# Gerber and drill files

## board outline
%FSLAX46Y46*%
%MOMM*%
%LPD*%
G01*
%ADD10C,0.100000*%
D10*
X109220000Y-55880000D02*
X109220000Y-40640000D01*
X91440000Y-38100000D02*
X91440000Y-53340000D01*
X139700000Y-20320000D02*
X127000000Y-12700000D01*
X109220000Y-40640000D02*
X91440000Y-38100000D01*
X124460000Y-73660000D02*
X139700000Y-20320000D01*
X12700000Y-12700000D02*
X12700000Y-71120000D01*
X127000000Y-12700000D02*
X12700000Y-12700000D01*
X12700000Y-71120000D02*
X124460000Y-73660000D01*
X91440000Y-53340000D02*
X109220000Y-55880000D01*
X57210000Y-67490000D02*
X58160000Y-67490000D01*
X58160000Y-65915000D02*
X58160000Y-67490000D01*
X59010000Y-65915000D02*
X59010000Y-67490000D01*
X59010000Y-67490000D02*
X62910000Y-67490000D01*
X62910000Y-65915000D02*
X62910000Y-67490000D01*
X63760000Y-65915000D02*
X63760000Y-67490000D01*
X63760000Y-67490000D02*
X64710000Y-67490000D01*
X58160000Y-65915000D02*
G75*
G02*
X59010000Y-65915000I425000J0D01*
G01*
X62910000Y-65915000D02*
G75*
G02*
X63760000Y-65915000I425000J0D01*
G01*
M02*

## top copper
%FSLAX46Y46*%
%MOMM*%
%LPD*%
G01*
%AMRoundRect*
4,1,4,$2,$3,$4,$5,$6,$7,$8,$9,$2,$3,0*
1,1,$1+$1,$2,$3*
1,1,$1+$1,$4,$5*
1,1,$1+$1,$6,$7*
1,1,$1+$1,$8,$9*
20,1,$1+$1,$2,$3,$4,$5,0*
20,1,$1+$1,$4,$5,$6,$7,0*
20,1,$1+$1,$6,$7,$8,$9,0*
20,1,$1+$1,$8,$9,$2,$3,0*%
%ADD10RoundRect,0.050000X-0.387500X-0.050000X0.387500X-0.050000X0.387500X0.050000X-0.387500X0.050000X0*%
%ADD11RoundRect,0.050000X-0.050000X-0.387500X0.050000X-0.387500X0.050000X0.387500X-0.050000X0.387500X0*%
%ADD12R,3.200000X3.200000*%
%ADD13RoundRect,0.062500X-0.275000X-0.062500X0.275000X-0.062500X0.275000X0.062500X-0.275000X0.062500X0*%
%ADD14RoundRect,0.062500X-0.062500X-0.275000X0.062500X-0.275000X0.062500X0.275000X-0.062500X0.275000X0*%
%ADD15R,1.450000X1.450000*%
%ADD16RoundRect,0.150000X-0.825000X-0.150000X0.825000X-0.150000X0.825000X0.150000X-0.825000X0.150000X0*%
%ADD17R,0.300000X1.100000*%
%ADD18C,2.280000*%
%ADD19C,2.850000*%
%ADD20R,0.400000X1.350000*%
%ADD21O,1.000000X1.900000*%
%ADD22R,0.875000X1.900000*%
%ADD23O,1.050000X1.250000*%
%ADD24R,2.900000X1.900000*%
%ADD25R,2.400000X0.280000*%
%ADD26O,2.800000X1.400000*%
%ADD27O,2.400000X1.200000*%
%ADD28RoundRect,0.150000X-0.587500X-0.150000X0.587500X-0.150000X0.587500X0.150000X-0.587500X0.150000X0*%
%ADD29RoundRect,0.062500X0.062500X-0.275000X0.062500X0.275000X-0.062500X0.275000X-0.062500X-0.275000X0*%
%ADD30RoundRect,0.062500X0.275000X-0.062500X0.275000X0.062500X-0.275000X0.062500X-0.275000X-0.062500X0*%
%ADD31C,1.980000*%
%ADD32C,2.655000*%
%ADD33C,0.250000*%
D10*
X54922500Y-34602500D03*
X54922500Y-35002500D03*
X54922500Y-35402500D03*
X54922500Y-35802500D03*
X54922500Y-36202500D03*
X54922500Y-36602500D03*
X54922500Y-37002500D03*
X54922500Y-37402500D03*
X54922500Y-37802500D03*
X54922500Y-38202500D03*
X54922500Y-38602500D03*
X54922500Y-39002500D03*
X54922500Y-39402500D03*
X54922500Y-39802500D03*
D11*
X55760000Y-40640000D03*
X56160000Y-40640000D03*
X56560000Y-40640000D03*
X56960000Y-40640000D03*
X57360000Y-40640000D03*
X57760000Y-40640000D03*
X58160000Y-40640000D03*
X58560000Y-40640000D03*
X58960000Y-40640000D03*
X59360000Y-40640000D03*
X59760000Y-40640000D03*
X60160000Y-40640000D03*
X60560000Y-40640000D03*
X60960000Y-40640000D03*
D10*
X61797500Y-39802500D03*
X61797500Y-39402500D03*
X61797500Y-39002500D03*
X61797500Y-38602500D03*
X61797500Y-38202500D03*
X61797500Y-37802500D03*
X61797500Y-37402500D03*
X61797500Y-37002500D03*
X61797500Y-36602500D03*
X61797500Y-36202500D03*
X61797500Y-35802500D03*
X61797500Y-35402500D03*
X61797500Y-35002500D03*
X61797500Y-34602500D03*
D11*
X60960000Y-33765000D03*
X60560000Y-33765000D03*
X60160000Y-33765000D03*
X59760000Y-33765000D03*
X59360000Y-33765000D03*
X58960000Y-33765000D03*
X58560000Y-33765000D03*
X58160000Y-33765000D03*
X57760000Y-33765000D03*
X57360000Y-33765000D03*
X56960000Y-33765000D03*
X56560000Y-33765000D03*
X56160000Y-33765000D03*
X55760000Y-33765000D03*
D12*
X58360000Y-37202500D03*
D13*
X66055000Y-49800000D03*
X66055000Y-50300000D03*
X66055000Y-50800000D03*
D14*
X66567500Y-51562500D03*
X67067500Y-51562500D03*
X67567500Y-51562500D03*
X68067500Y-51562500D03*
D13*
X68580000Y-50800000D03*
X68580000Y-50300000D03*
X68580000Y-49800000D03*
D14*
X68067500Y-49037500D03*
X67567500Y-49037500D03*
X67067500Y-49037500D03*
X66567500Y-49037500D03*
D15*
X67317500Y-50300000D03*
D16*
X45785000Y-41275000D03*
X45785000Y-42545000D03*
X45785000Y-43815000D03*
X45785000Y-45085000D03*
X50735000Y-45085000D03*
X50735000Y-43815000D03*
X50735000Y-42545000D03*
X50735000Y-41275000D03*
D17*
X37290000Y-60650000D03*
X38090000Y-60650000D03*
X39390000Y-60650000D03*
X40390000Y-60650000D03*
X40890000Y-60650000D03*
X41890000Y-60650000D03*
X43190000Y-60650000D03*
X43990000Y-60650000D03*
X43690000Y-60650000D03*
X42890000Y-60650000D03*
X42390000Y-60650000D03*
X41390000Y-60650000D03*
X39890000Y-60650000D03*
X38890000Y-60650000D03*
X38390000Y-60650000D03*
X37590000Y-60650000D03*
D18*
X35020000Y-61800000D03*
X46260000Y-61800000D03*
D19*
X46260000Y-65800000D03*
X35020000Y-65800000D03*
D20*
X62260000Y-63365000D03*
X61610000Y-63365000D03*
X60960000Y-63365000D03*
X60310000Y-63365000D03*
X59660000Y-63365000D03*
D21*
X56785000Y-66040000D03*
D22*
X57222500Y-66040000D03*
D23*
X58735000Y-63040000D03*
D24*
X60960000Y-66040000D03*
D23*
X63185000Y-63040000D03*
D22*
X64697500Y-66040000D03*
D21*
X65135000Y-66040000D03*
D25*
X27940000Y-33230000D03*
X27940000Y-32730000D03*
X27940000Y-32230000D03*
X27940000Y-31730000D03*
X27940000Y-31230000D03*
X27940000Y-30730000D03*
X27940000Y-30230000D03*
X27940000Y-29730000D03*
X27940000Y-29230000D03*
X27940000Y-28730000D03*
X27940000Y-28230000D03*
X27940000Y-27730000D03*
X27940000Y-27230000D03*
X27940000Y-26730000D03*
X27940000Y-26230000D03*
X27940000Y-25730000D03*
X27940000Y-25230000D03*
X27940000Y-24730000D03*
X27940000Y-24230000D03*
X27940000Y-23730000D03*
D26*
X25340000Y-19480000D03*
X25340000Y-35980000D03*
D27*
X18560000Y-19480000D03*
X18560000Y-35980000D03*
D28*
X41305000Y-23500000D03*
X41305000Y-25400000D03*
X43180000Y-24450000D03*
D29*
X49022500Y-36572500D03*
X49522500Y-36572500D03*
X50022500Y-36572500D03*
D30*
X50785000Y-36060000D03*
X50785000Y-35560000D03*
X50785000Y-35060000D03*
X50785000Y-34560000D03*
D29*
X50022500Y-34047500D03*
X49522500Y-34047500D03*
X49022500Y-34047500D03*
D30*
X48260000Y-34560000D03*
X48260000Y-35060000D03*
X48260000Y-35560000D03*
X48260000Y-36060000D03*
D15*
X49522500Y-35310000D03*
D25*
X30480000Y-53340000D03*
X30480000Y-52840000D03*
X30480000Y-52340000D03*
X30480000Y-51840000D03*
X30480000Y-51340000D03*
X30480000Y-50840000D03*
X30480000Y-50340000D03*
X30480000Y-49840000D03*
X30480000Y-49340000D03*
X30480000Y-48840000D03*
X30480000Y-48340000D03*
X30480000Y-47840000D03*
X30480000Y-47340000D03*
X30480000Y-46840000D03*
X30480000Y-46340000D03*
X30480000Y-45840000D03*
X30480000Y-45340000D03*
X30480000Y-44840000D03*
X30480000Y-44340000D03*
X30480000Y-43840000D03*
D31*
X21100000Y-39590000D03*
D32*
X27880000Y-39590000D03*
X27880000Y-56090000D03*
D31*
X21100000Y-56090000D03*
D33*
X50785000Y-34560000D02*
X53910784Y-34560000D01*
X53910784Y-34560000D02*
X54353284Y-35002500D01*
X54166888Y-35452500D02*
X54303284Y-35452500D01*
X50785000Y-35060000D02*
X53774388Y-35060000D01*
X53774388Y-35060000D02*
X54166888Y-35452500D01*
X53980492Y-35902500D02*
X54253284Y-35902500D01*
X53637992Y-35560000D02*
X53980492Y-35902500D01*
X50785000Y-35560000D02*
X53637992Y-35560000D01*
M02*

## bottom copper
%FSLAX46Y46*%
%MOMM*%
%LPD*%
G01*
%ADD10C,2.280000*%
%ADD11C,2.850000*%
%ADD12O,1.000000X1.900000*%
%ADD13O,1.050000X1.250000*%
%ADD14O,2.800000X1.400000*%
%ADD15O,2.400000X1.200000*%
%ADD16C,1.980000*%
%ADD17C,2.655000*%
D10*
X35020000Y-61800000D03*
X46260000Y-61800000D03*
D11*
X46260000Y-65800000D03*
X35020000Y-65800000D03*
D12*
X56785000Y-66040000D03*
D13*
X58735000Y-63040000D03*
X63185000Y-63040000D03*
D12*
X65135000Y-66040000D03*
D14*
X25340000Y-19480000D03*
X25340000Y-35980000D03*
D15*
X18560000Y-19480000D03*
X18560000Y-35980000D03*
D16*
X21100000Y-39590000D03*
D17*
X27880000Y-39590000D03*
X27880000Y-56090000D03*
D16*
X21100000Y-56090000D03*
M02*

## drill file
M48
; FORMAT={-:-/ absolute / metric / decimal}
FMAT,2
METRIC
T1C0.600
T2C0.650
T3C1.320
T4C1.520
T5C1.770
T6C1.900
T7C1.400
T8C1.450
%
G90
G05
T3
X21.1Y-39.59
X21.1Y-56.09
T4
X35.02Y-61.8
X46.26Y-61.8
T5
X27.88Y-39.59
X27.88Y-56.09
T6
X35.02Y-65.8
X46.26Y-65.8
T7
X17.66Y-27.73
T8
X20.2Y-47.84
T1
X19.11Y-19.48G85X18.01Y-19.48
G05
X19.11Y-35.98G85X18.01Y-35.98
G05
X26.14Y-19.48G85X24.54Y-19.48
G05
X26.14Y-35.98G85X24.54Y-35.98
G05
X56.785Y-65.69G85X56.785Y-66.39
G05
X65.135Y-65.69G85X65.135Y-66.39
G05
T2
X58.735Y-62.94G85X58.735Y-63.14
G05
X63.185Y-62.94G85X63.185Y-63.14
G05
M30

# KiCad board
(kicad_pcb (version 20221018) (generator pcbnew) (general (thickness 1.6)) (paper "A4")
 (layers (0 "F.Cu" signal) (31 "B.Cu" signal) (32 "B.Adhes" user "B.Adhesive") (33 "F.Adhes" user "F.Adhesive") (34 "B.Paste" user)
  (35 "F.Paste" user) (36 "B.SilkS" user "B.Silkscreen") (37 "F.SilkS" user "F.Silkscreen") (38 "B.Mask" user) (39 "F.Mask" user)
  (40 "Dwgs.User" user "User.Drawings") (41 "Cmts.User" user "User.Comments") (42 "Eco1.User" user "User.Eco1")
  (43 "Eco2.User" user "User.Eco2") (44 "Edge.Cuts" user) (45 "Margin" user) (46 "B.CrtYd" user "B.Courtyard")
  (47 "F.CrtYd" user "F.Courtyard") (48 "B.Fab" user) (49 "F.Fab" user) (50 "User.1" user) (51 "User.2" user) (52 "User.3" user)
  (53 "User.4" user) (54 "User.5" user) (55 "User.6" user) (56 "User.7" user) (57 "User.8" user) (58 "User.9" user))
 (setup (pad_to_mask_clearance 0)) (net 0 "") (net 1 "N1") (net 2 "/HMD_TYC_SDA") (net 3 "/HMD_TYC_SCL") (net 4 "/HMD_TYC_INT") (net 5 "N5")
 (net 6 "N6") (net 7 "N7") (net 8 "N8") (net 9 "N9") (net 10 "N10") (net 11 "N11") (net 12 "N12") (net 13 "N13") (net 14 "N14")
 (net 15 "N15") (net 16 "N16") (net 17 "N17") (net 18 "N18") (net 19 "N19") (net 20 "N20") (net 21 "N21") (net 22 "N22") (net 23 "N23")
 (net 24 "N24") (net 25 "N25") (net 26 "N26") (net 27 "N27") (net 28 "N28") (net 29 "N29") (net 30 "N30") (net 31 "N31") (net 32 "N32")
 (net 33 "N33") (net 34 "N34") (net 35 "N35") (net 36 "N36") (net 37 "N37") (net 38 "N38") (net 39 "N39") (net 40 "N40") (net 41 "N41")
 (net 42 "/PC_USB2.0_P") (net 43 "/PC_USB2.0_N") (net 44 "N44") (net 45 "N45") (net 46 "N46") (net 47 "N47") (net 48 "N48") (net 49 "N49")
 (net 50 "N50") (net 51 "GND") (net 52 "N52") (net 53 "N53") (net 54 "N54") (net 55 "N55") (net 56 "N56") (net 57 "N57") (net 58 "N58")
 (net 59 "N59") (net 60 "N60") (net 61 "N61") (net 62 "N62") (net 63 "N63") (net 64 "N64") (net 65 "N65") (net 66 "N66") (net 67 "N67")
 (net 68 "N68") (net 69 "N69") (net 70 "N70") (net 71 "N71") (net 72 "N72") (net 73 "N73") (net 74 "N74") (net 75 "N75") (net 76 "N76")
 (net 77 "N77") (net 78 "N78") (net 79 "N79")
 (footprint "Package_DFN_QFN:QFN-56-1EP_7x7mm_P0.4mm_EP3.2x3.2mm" (layer "F.Cu") (at 58.36 37.2025)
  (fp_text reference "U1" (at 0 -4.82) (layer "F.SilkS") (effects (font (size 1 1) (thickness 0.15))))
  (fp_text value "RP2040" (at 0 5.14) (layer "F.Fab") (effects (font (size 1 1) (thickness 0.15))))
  (pad "" smd roundrect (at -0.8 -0.8) (size 1.29 1.29) (layers "F.Paste") (roundrect_rratio 0.193798))
  (pad "" smd roundrect (at -0.8 0.8) (size 1.29 1.29) (layers "F.Paste") (roundrect_rratio 0.193798))
  (pad "" smd roundrect (at 0.8 -0.8) (size 1.29 1.29) (layers "F.Paste") (roundrect_rratio 0.193798))
  (pad "" smd roundrect (at 0.8 0.8) (size 1.29 1.29) (layers "F.Paste") (roundrect_rratio 0.193798))
  (pad "1" smd roundrect (at -3.4375 -2.6) (size 0.875 0.2) (layers "F.Cu" "F.Paste" "F.Mask") (roundrect_rratio 0.25) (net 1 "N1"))
  (pad "2" smd roundrect (at -3.4375 -2.2) (size 0.875 0.2) (layers "F.Cu" "F.Paste" "F.Mask") (roundrect_rratio 0.25)
   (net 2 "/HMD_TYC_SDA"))
  (pad "3" smd roundrect (at -3.4375 -1.8) (size 0.875 0.2) (layers "F.Cu" "F.Paste" "F.Mask") (roundrect_rratio 0.25)
   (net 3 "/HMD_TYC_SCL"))
  (pad "4" smd roundrect (at -3.4375 -1.4) (size 0.875 0.2) (layers "F.Cu" "F.Paste" "F.Mask") (roundrect_rratio 0.25)
   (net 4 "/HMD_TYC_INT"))
  (pad "5" smd roundrect (at -3.4375 -1) (size 0.875 0.2) (layers "F.Cu" "F.Paste" "F.Mask") (roundrect_rratio 0.25) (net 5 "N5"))
  (pad "6" smd roundrect (at -3.4375 -0.6) (size 0.875 0.2) (layers "F.Cu" "F.Paste" "F.Mask") (roundrect_rratio 0.25) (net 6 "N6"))
  (pad "7" smd roundrect (at -3.4375 -0.2) (size 0.875 0.2) (layers "F.Cu" "F.Paste" "F.Mask") (roundrect_rratio 0.25) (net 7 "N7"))
  (pad "8" smd roundrect (at -3.4375 0.2) (size 0.875 0.2) (layers "F.Cu" "F.Paste" "F.Mask") (roundrect_rratio 0.25) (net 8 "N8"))
  (pad "9" smd roundrect (at -3.4375 0.6) (size 0.875 0.2) (layers "F.Cu" "F.Paste" "F.Mask") (roundrect_rratio 0.25) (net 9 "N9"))
  (pad "10" smd roundrect (at -3.4375 1) (size 0.875 0.2) (layers "F.Cu" "F.Paste" "F.Mask") (roundrect_rratio 0.25) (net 1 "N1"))
  (pad "11" smd roundrect (at -3.4375 1.4) (size 0.875 0.2) (layers "F.Cu" "F.Paste" "F.Mask") (roundrect_rratio 0.25) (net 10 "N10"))
  (pad "12" smd roundrect (at -3.4375 1.8) (size 0.875 0.2) (layers "F.Cu" "F.Paste" "F.Mask") (roundrect_rratio 0.25) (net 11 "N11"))
  (pad "13" smd roundrect (at -3.4375 2.2) (size 0.875 0.2) (layers "F.Cu" "F.Paste" "F.Mask") (roundrect_rratio 0.25) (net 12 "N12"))
  (pad "14" smd roundrect (at -3.4375 2.6) (size 0.875 0.2) (layers "F.Cu" "F.Paste" "F.Mask") (roundrect_rratio 0.25) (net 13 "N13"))
  (pad "15" smd roundrect (at -2.6 3.4375) (size 0.2 0.875) (layers "F.Cu" "F.Paste" "F.Mask") (roundrect_rratio 0.25) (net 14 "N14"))
  (pad "16" smd roundrect (at -2.2 3.4375) (size 0.2 0.875) (layers "F.Cu" "F.Paste" "F.Mask") (roundrect_rratio 0.25) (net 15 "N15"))
  (pad "17" smd roundrect (at -1.8 3.4375) (size 0.2 0.875) (layers "F.Cu" "F.Paste" "F.Mask") (roundrect_rratio 0.25) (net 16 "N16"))
  (pad "18" smd roundrect (at -1.4 3.4375) (size 0.2 0.875) (layers "F.Cu" "F.Paste" "F.Mask") (roundrect_rratio 0.25) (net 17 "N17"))
  (pad "19" smd roundrect (at -1 3.4375) (size 0.2 0.875) (layers "F.Cu" "F.Paste" "F.Mask") (roundrect_rratio 0.25) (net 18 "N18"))
  (pad "20" smd roundrect (at -0.6 3.4375) (size 0.2 0.875) (layers "F.Cu" "F.Paste" "F.Mask") (roundrect_rratio 0.25) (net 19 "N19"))
  (pad "21" smd roundrect (at -0.2 3.4375) (size 0.2 0.875) (layers "F.Cu" "F.Paste" "F.Mask") (roundrect_rratio 0.25) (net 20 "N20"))
  (pad "22" smd roundrect (at 0.2 3.4375) (size 0.2 0.875) (layers "F.Cu" "F.Paste" "F.Mask") (roundrect_rratio 0.25) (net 1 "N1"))
  (pad "23" smd roundrect (at 0.6 3.4375) (size 0.2 0.875) (layers "F.Cu" "F.Paste" "F.Mask") (roundrect_rratio 0.25) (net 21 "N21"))
  (pad "24" smd roundrect (at 1 3.4375) (size 0.2 0.875) (layers "F.Cu" "F.Paste" "F.Mask") (roundrect_rratio 0.25) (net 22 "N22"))
  (pad "25" smd roundrect (at 1.4 3.4375) (size 0.2 0.875) (layers "F.Cu" "F.Paste" "F.Mask") (roundrect_rratio 0.25) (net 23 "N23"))
  (pad "26" smd roundrect (at 1.8 3.4375) (size 0.2 0.875) (layers "F.Cu" "F.Paste" "F.Mask") (roundrect_rratio 0.25) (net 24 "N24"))
  (pad "27" smd roundrect (at 2.2 3.4375) (size 0.2 0.875) (layers "F.Cu" "F.Paste" "F.Mask") (roundrect_rratio 0.25) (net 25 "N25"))
  (pad "28" smd roundrect (at 2.6 3.4375) (size 0.2 0.875) (layers "F.Cu" "F.Paste" "F.Mask") (roundrect_rratio 0.25) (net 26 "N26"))
  (pad "29" smd roundrect (at 3.4375 2.6) (size 0.875 0.2) (layers "F.Cu" "F.Paste" "F.Mask") (roundrect_rratio 0.25) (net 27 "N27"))
  (pad "30" smd roundrect (at 3.4375 2.2) (size 0.875 0.2) (layers "F.Cu" "F.Paste" "F.Mask") (roundrect_rratio 0.25) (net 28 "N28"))
  (pad "31" smd roundrect (at 3.4375 1.8) (size 0.875 0.2) (layers "F.Cu" "F.Paste" "F.Mask") (roundrect_rratio 0.25) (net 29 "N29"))
  (pad "32" smd roundrect (at 3.4375 1.4) (size 0.875 0.2) (layers "F.Cu" "F.Paste" "F.Mask") (roundrect_rratio 0.25) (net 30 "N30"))
  (pad "33" smd roundrect (at 3.4375 1) (size 0.875 0.2) (layers "F.Cu" "F.Paste" "F.Mask") (roundrect_rratio 0.25) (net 1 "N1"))
  (pad "34" smd roundrect (at 3.4375 0.6) (size 0.875 0.2) (layers "F.Cu" "F.Paste" "F.Mask") (roundrect_rratio 0.25) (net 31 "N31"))
  (pad "35" smd roundrect (at 3.4375 0.2) (size 0.875 0.2) (layers "F.Cu" "F.Paste" "F.Mask") (roundrect_rratio 0.25) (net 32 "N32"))
  (pad "36" smd roundrect (at 3.4375 -0.2) (size 0.875 0.2) (layers "F.Cu" "F.Paste" "F.Mask") (roundrect_rratio 0.25) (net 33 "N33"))
  (pad "37" smd roundrect (at 3.4375 -0.6) (size 0.875 0.2) (layers "F.Cu" "F.Paste" "F.Mask") (roundrect_rratio 0.25) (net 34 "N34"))
  (pad "38" smd roundrect (at 3.4375 -1) (size 0.875 0.2) (layers "F.Cu" "F.Paste" "F.Mask") (roundrect_rratio 0.25) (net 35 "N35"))
  (pad "39" smd roundrect (at 3.4375 -1.4) (size 0.875 0.2) (layers "F.Cu" "F.Paste" "F.Mask") (roundrect_rratio 0.25) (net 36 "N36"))
  (pad "40" smd roundrect (at 3.4375 -1.8) (size 0.875 0.2) (layers "F.Cu" "F.Paste" "F.Mask") (roundrect_rratio 0.25) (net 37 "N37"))
  (pad "41" smd roundrect (at 3.4375 -2.2) (size 0.875 0.2) (layers "F.Cu" "F.Paste" "F.Mask") (roundrect_rratio 0.25) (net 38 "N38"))
  (pad "42" smd roundrect (at 3.4375 -2.6) (size 0.875 0.2) (layers "F.Cu" "F.Paste" "F.Mask") (roundrect_rratio 0.25) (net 1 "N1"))
  (pad "43" smd roundrect (at 2.6 -3.4375) (size 0.2 0.875) (layers "F.Cu" "F.Paste" "F.Mask") (roundrect_rratio 0.25) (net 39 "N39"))
  (pad "44" smd roundrect (at 2.2 -3.4375) (size 0.2 0.875) (layers "F.Cu" "F.Paste" "F.Mask") (roundrect_rratio 0.25) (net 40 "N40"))
  (pad "45" smd roundrect (at 1.8 -3.4375) (size 0.2 0.875) (layers "F.Cu" "F.Paste" "F.Mask") (roundrect_rratio 0.25) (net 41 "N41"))
  (pad "46" smd roundrect (at 1.4 -3.4375) (size 0.2 0.875) (layers "F.Cu" "F.Paste" "F.Mask") (roundrect_rratio 0.25)
   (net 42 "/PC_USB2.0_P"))
  (pad "47" smd roundrect (at 1 -3.4375) (size 0.2 0.875) (layers "F.Cu" "F.Paste" "F.Mask") (roundrect_rratio 0.25) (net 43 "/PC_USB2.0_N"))
  (pad "48" smd roundrect (at 0.6 -3.4375) (size 0.2 0.875) (layers "F.Cu" "F.Paste" "F.Mask") (roundrect_rratio 0.25) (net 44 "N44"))
  (pad "49" smd roundrect (at 0.2 -3.4375) (size 0.2 0.875) (layers "F.Cu" "F.Paste" "F.Mask") (roundrect_rratio 0.25) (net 1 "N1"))
  (pad "50" smd roundrect (at -0.2 -3.4375) (size 0.2 0.875) (layers "F.Cu" "F.Paste" "F.Mask") (roundrect_rratio 0.25) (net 21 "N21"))
  (pad "51" smd roundrect (at -0.6 -3.4375) (size 0.2 0.875) (layers "F.Cu" "F.Paste" "F.Mask") (roundrect_rratio 0.25) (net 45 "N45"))
  (pad "52" smd roundrect (at -1 -3.4375) (size 0.2 0.875) (layers "F.Cu" "F.Paste" "F.Mask") (roundrect_rratio 0.25) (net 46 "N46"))
  (pad "53" smd roundrect (at -1.4 -3.4375) (size 0.2 0.875) (layers "F.Cu" "F.Paste" "F.Mask") (roundrect_rratio 0.25) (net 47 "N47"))
  (pad "54" smd roundrect (at -1.8 -3.4375) (size 0.2 0.875) (layers "F.Cu" "F.Paste" "F.Mask") (roundrect_rratio 0.25) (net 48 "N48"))
  (pad "55" smd roundrect (at -2.2 -3.4375) (size 0.2 0.875) (layers "F.Cu" "F.Paste" "F.Mask") (roundrect_rratio 0.25) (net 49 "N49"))
  (pad "56" smd roundrect (at -2.6 -3.4375) (size 0.2 0.875) (layers "F.Cu" "F.Paste" "F.Mask") (roundrect_rratio 0.25) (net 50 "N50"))
  (pad "57" smd rect (at 0 0) (size 3.2 3.2) (layers "F.Cu" "F.Mask") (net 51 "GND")))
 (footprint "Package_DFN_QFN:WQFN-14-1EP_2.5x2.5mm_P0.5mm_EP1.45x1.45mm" (layer "F.Cu") (at 67.3175 50.3)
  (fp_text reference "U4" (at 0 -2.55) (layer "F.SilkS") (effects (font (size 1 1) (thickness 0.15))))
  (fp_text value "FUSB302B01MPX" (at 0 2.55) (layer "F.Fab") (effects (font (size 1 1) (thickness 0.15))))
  (pad "" smd roundrect (at -0.36 -0.36) (size 0.58 0.58) (layers "F.Paste") (roundrect_rratio 0.25))
  (pad "" smd roundrect (at -0.36 0.36) (size 0.58 0.58) (layers "F.Paste") (roundrect_rratio 0.25))
  (pad "" smd roundrect (at 0.36 -0.36) (size 0.58 0.58) (layers "F.Paste") (roundrect_rratio 0.25))
  (pad "" smd roundrect (at 0.36 0.36) (size 0.58 0.58) (layers "F.Paste") (roundrect_rratio 0.25))
  (pad "1" smd roundrect (at -1.2625 -0.5) (size 0.675 0.25) (layers "F.Cu" "F.Paste" "F.Mask") (roundrect_rratio 0.25) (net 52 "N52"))
  (pad "2" smd roundrect (at -1.2625 0) (size 0.675 0.25) (layers "F.Cu" "F.Paste" "F.Mask") (roundrect_rratio 0.25) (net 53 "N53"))
  (pad "3" smd roundrect (at -1.2625 0.5) (size 0.675 0.25) (layers "F.Cu" "F.Paste" "F.Mask") (roundrect_rratio 0.25) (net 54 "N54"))
  (pad "4" smd roundrect (at -0.75 1.2625) (size 0.25 0.675) (layers "F.Cu" "F.Paste" "F.Mask") (roundrect_rratio 0.25) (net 54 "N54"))
  (pad "5" smd roundrect (at -0.25 1.2625) (size 0.25 0.675) (layers "F.Cu" "F.Paste" "F.Mask") (roundrect_rratio 0.25) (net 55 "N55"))
  (pad "6" smd roundrect (at 0.25 1.2625) (size 0.25 0.675) (layers "F.Cu" "F.Paste" "F.Mask") (roundrect_rratio 0.25) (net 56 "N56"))
  (pad "7" smd roundrect (at 0.75 1.2625) (size 0.25 0.675) (layers "F.Cu" "F.Paste" "F.Mask") (roundrect_rratio 0.25) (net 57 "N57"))
  (pad "8" smd roundrect (at 1.2625 0.5) (size 0.675 0.25) (layers "F.Cu" "F.Paste" "F.Mask") (roundrect_rratio 0.25) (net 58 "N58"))
  (pad "9" smd roundrect (at 1.2625 0) (size 0.675 0.25) (layers "F.Cu" "F.Paste" "F.Mask") (roundrect_rratio 0.25) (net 58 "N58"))
  (pad "10" smd roundrect (at 1.2625 -0.5) (size 0.675 0.25) (layers "F.Cu" "F.Paste" "F.Mask") (roundrect_rratio 0.25) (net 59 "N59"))
  (pad "11" smd roundrect (at 0.75 -1.2625) (size 0.25 0.675) (layers "F.Cu" "F.Paste" "F.Mask") (roundrect_rratio 0.25) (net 59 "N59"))
  (pad "12" smd roundrect (at 0.25 -1.2625) (size 0.25 0.675) (layers "F.Cu" "F.Paste" "F.Mask") (roundrect_rratio 0.25) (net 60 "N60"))
  (pad "13" smd roundrect (at -0.25 -1.2625) (size 0.25 0.675) (layers "F.Cu" "F.Paste" "F.Mask") (roundrect_rratio 0.25) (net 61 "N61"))
  (pad "14" smd roundrect (at -0.75 -1.2625) (size 0.25 0.675) (layers "F.Cu" "F.Paste" "F.Mask") (roundrect_rratio 0.25) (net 52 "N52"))
  (pad "15" smd rect (at 0 0) (size 1.45 1.45) (layers "F.Cu" "F.Mask") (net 58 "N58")))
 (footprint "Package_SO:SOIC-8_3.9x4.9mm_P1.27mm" (layer "F.Cu") (at 48.26 43.18)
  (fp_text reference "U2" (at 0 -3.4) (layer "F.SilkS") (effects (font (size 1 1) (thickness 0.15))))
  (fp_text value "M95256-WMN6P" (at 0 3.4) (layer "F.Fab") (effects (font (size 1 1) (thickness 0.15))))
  (pad "1" smd roundrect (at -2.475 -1.905) (size 1.95 0.6) (layers "F.Cu" "F.Paste" "F.Mask") (roundrect_rratio 0.25) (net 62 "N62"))
  (pad "2" smd roundrect (at -2.475 -0.635) (size 1.95 0.6) (layers "F.Cu" "F.Paste" "F.Mask") (roundrect_rratio 0.25) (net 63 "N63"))
  (pad "3" smd roundrect (at -2.475 0.635) (size 1.95 0.6) (layers "F.Cu" "F.Paste" "F.Mask") (roundrect_rratio 0.25) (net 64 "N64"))
  (pad "4" smd roundrect (at -2.475 1.905) (size 1.95 0.6) (layers "F.Cu" "F.Paste" "F.Mask") (roundrect_rratio 0.25) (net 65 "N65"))
  (pad "5" smd roundrect (at 2.475 1.905) (size 1.95 0.6) (layers "F.Cu" "F.Paste" "F.Mask") (roundrect_rratio 0.25) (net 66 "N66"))
  (pad "6" smd roundrect (at 2.475 0.635) (size 1.95 0.6) (layers "F.Cu" "F.Paste" "F.Mask") (roundrect_rratio 0.25) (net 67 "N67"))
  (pad "7" smd roundrect (at 2.475 -0.635) (size 1.95 0.6) (layers "F.Cu" "F.Paste" "F.Mask") (roundrect_rratio 0.25) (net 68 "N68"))
  (pad "8" smd roundrect (at 2.475 -1.905) (size 1.95 0.6) (layers "F.Cu" "F.Paste" "F.Mask") (roundrect_rratio 0.25) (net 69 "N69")))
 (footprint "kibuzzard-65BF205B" (layer "F.Cu") (at 88.9 27.94)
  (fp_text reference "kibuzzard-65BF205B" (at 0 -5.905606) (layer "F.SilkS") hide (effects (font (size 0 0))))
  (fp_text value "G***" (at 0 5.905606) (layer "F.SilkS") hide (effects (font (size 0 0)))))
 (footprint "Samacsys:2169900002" (layer "F.Cu") (at 40.64 63.5)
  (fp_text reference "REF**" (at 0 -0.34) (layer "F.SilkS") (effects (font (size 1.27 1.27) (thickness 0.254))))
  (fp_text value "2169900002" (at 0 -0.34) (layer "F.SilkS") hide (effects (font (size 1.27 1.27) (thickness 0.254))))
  (pad "A1" smd rect (at -3.35 -2.85) (size 0.3 1.1) (layers "F.Cu" "F.Paste" "F.Mask"))
  (pad "A4" smd rect (at -2.55 -2.85) (size 0.3 1.1) (layers "F.Cu" "F.Paste" "F.Mask"))
  (pad "A5" smd rect (at -1.25 -2.85) (size 0.3 1.1) (layers "F.Cu" "F.Paste" "F.Mask"))
  (pad "A6" smd rect (at -0.25 -2.85) (size 0.3 1.1) (layers "F.Cu" "F.Paste" "F.Mask"))
  (pad "A7" smd rect (at 0.25 -2.85) (size 0.3 1.1) (layers "F.Cu" "F.Paste" "F.Mask"))
  (pad "A8" smd rect (at 1.25 -2.85) (size 0.3 1.1) (layers "F.Cu" "F.Paste" "F.Mask"))
  (pad "A9" smd rect (at 2.55 -2.85) (size 0.3 1.1) (layers "F.Cu" "F.Paste" "F.Mask"))
  (pad "A12" smd rect (at 3.35 -2.85) (size 0.3 1.1) (layers "F.Cu" "F.Paste" "F.Mask"))
  (pad "B1" smd rect (at 3.05 -2.85) (size 0.3 1.1) (layers "F.Cu" "F.Paste" "F.Mask"))
  (pad "B4" smd rect (at 2.25 -2.85) (size 0.3 1.1) (layers "F.Cu" "F.Paste" "F.Mask"))
  (pad "B5" smd rect (at 1.75 -2.85) (size 0.3 1.1) (layers "F.Cu" "F.Paste" "F.Mask"))
  (pad "B6" smd rect (at 0.75 -2.85) (size 0.3 1.1) (layers "F.Cu" "F.Paste" "F.Mask"))
  (pad "B7" smd rect (at -0.75 -2.85) (size 0.3 1.1) (layers "F.Cu" "F.Paste" "F.Mask"))
  (pad "B8" smd rect (at -1.75 -2.85) (size 0.3 1.1) (layers "F.Cu" "F.Paste" "F.Mask"))
  (pad "B9" smd rect (at -2.25 -2.85) (size 0.3 1.1) (layers "F.Cu" "F.Paste" "F.Mask"))
  (pad "B12" smd rect (at -3.05 -2.85) (size 0.3 1.1) (layers "F.Cu" "F.Paste" "F.Mask"))
  (pad "MH1" thru_hole circle (at -5.62 -1.7) (size 2.28 2.28) (drill 1.52) (layers "*.Cu" "*.Mask"))
  (pad "MH2" thru_hole circle (at 5.62 -1.7) (size 2.28 2.28) (drill 1.52) (layers "*.Cu" "*.Mask"))
  (pad "MH3" thru_hole circle (at 5.62 2.3) (size 2.85 2.85) (drill 1.9) (layers "*.Cu" "*.Mask"))
  (pad "MH4" thru_hole circle (at -5.62 2.3) (size 2.85 2.85) (drill 1.9) (layers "*.Cu" "*.Mask")))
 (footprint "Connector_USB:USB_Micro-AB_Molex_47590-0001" (layer "F.Cu") (at 60.96 66.04)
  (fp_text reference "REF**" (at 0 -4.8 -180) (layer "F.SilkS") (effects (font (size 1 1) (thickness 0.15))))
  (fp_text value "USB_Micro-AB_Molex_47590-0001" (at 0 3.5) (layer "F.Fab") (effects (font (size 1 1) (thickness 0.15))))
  (fp_line (start -3.75 1.45) (end -2.8 1.45) (stroke (width 0.1) (type solid)) (layer "Edge.Cuts"))
  (fp_line (start -2.8 -0.125) (end -2.8 1.45) (stroke (width 0.1) (type solid)) (layer "Edge.Cuts"))
  (fp_line (start -1.95 -0.125) (end -1.95 1.45) (stroke (width 0.1) (type solid)) (layer "Edge.Cuts"))
  (fp_line (start -1.95 1.45) (end 1.95 1.45) (stroke (width 0.1) (type solid)) (layer "Edge.Cuts"))
  (fp_line (start 1.95 -0.125) (end 1.95 1.45) (stroke (width 0.1) (type solid)) (layer "Edge.Cuts"))
  (fp_line (start 2.8 -0.125) (end 2.8 1.45) (stroke (width 0.1) (type solid)) (layer "Edge.Cuts"))
  (fp_line (start 2.8 1.45) (end 3.75 1.45) (stroke (width 0.1) (type solid)) (layer "Edge.Cuts"))
  (fp_arc (start -2.8 -0.125) (mid -2.375 -0.55) (end -1.95 -0.125) (stroke (width 0.1) (type solid)) (layer "Edge.Cuts"))
  (fp_arc (start 1.95 -0.125) (mid 2.375 -0.55) (end 2.8 -0.125) (stroke (width 0.1) (type solid)) (layer "Edge.Cuts"))
  (pad "" smd rect (at -3.5 0) (size 0.3 0.85) (layers "F.Paste"))
  (pad "" smd rect (at 3.5 0) (size 0.3 0.85) (layers "F.Paste"))
  (pad "1" smd rect (at 1.3 -2.675) (size 0.4 1.35) (layers "F.Cu" "F.Paste" "F.Mask"))
  (pad "2" smd rect (at 0.65 -2.675) (size 0.4 1.35) (layers "F.Cu" "F.Paste" "F.Mask"))
  (pad "3" smd rect (at 0 -2.675) (size 0.4 1.35) (layers "F.Cu" "F.Paste" "F.Mask"))
  (pad "4" smd rect (at -0.65 -2.675) (size 0.4 1.35) (layers "F.Cu" "F.Paste" "F.Mask"))
  (pad "5" smd rect (at -1.3 -2.675) (size 0.4 1.35) (layers "F.Cu" "F.Paste" "F.Mask"))
  (pad "6" thru_hole oval (at -4.175 0) (size 1 1.9) (drill oval 0.6 1.3) (layers "*.Cu" "*.Mask"))
  (pad "6" smd rect (at -3.7375 0) (size 0.875 1.9) (layers "F.Cu" "F.Mask"))
  (pad "6" thru_hole oval (at -2.225 -3) (size 1.05 1.25) (drill oval 0.65 0.85) (layers "*.Cu" "*.Mask"))
  (pad "6" smd rect (at 0 0) (size 2.9 1.9) (layers "F.Cu" "F.Paste" "F.Mask"))
  (pad "6" thru_hole oval (at 2.225 -3) (size 1.05 1.25) (drill oval 0.65 0.85) (layers "*.Cu" "*.Mask"))
  (pad "6" smd rect (at 3.7375 0) (size 0.875 1.9) (layers "F.Cu" "F.Mask"))
  (pad "6" thru_hole oval (at 4.175 0) (size 1 1.9) (drill oval 0.6 1.3) (layers "*.Cu" "*.Mask")))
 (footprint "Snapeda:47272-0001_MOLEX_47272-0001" (layer "F.Cu") (at 14.38 27.73 -90)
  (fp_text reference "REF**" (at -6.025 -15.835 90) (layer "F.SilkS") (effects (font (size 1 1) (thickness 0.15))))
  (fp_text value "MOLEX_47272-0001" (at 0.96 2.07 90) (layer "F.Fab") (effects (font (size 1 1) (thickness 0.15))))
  (pad "" np_thru_hole circle (at 0 -3.28 270) (size 1.4 1.4) (drill 1.4) (layers "*.Cu" "*.Mask"))
  (pad "1" smd rect (at 5.5 -13.56) (size 2.4 0.28) (layers "F.Cu" "F.Paste" "F.Mask") (solder_mask_margin 0.0762))
  (pad "2" smd rect (at 5 -13.56) (size 2.4 0.28) (layers "F.Cu" "F.Paste" "F.Mask") (solder_mask_margin 0.0762))
  (pad "3" smd rect (at 4.5 -13.56) (size 2.4 0.28) (layers "F.Cu" "F.Paste" "F.Mask") (solder_mask_margin 0.0762))
  (pad "4" smd rect (at 4 -13.56) (size 2.4 0.28) (layers "F.Cu" "F.Paste" "F.Mask") (solder_mask_margin 0.0762))
  (pad "5" smd rect (at 3.5 -13.56) (size 2.4 0.28) (layers "F.Cu" "F.Paste" "F.Mask") (solder_mask_margin 0.0762))
  (pad "6" smd rect (at 3 -13.56) (size 2.4 0.28) (layers "F.Cu" "F.Paste" "F.Mask") (solder_mask_margin 0.0762))
  (pad "7" smd rect (at 2.5 -13.56) (size 2.4 0.28) (layers "F.Cu" "F.Paste" "F.Mask") (solder_mask_margin 0.0762))
  (pad "8" smd rect (at 2 -13.56) (size 2.4 0.28) (layers "F.Cu" "F.Paste" "F.Mask") (solder_mask_margin 0.0762))
  (pad "9" smd rect (at 1.5 -13.56) (size 2.4 0.28) (layers "F.Cu" "F.Paste" "F.Mask") (solder_mask_margin 0.0762))
  (pad "10" smd rect (at 1 -13.56) (size 2.4 0.28) (layers "F.Cu" "F.Paste" "F.Mask") (solder_mask_margin 0.0762))
  (pad "11" smd rect (at 0.5 -13.56) (size 2.4 0.28) (layers "F.Cu" "F.Paste" "F.Mask") (solder_mask_margin 0.0762))
  (pad "12" smd rect (at 0 -13.56) (size 2.4 0.28) (layers "F.Cu" "F.Paste" "F.Mask") (solder_mask_margin 0.0762))
  (pad "13" smd rect (at -0.5 -13.56) (size 2.4 0.28) (layers "F.Cu" "F.Paste" "F.Mask") (solder_mask_margin 0.0762))
  (pad "14" smd rect (at -1 -13.56) (size 2.4 0.28) (layers "F.Cu" "F.Paste" "F.Mask") (solder_mask_margin 0.0762))
  (pad "15" smd rect (at -1.5 -13.56) (size 2.4 0.28) (layers "F.Cu" "F.Paste" "F.Mask") (solder_mask_margin 0.0762))
  (pad "16" smd rect (at -2 -13.56) (size 2.4 0.28) (layers "F.Cu" "F.Paste" "F.Mask") (solder_mask_margin 0.0762))
  (pad "17" smd rect (at -2.5 -13.56) (size 2.4 0.28) (layers "F.Cu" "F.Paste" "F.Mask") (solder_mask_margin 0.0762))
  (pad "18" smd rect (at -3 -13.56) (size 2.4 0.28) (layers "F.Cu" "F.Paste" "F.Mask") (solder_mask_margin 0.0762))
  (pad "19" smd rect (at -3.5 -13.56) (size 2.4 0.28) (layers "F.Cu" "F.Paste" "F.Mask") (solder_mask_margin 0.0762))
  (pad "20" smd rect (at -4 -13.56) (size 2.4 0.28) (layers "F.Cu" "F.Paste" "F.Mask") (solder_mask_margin 0.0762))
  (pad "S1" thru_hole oval (at -8.25 -10.96 270) (size 1.4 2.8) (drill oval 0.6 2.2) (layers "*.Cu" "*.Mask") (solder_mask_margin 0.0762))
  (pad "S2" thru_hole oval (at 8.25 -10.96 270) (size 1.4 2.8) (drill oval 0.6 2.2) (layers "*.Cu" "*.Mask") (solder_mask_margin 0.0762))
  (pad "S3" thru_hole oval (at -8.25 -4.18 270) (size 1.2 2.4) (drill oval 0.6 1.7) (layers "*.Cu" "*.Mask") (solder_mask_margin 0.0762))
  (pad "S4" thru_hole oval (at 8.25 -4.18 270) (size 1.2 2.4) (drill oval 0.6 1.7) (layers "*.Cu" "*.Mask") (solder_mask_margin 0.0762)))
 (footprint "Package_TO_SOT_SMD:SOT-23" (layer "F.Cu") (at 42.2425 24.45)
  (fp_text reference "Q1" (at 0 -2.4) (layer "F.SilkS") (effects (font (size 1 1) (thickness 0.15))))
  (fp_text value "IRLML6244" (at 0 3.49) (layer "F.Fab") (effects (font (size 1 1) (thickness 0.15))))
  (pad "1" smd roundrect (at -0.9375 -0.95) (size 1.475 0.6) (layers "F.Cu" "F.Paste" "F.Mask") (roundrect_rratio 0.25) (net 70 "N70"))
  (pad "2" smd roundrect (at -0.9375 0.95) (size 1.475 0.6) (layers "F.Cu" "F.Paste" "F.Mask") (roundrect_rratio 0.25) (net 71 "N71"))
  (pad "3" smd roundrect (at 0.9375 0) (size 1.475 0.6) (layers "F.Cu" "F.Paste" "F.Mask") (roundrect_rratio 0.25) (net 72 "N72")))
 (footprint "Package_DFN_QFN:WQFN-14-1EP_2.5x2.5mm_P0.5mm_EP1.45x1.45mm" (layer "F.Cu") (at 49.5225 35.31 90)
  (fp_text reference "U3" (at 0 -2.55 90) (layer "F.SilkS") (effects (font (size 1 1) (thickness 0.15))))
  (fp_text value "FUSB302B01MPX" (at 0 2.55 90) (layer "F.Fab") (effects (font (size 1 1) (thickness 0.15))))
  (pad "" smd roundrect (at -0.36 -0.36 90) (size 0.58 0.58) (layers "F.Paste") (roundrect_rratio 0.25))
  (pad "" smd roundrect (at -0.36 0.36 90) (size 0.58 0.58) (layers "F.Paste") (roundrect_rratio 0.25))
  (pad "" smd roundrect (at 0.36 -0.36 90) (size 0.58 0.58) (layers "F.Paste") (roundrect_rratio 0.25))
  (pad "" smd roundrect (at 0.36 0.36 90) (size 0.58 0.58) (layers "F.Paste") (roundrect_rratio 0.25))
  (pad "1" smd roundrect (at -1.2625 -0.5 90) (size 0.675 0.25) (layers "F.Cu" "F.Paste" "F.Mask") (roundrect_rratio 0.25) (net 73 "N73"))
  (pad "2" smd roundrect (at -1.2625 0 90) (size 0.675 0.25) (layers "F.Cu" "F.Paste" "F.Mask") (roundrect_rratio 0.25) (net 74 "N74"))
  (pad "3" smd roundrect (at -1.2625 0.5 90) (size 0.675 0.25) (layers "F.Cu" "F.Paste" "F.Mask") (roundrect_rratio 0.25) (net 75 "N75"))
  (pad "4" smd roundrect (at -0.75 1.2625 90) (size 0.25 0.675) (layers "F.Cu" "F.Paste" "F.Mask") (roundrect_rratio 0.25) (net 75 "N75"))
  (pad "5" smd roundrect (at -0.25 1.2625 90) (size 0.25 0.675) (layers "F.Cu" "F.Paste" "F.Mask") (roundrect_rratio 0.25)
   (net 4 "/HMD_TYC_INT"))
  (pad "6" smd roundrect (at 0.25 1.2625 90) (size 0.25 0.675) (layers "F.Cu" "F.Paste" "F.Mask") (roundrect_rratio 0.25)
   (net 3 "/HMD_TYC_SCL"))
  (pad "7" smd roundrect (at 0.75 1.2625 90) (size 0.25 0.675) (layers "F.Cu" "F.Paste" "F.Mask") (roundrect_rratio 0.25)
   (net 2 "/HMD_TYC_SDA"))
  (pad "8" smd roundrect (at 1.2625 0.5 90) (size 0.675 0.25) (layers "F.Cu" "F.Paste" "F.Mask") (roundrect_rratio 0.25) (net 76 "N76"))
  (pad "9" smd roundrect (at 1.2625 0 90) (size 0.675 0.25) (layers "F.Cu" "F.Paste" "F.Mask") (roundrect_rratio 0.25) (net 76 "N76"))
  (pad "10" smd roundrect (at 1.2625 -0.5 90) (size 0.675 0.25) (layers "F.Cu" "F.Paste" "F.Mask") (roundrect_rratio 0.25) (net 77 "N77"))
  (pad "11" smd roundrect (at 0.75 -1.2625 90) (size 0.25 0.675) (layers "F.Cu" "F.Paste" "F.Mask") (roundrect_rratio 0.25) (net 77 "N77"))
  (pad "12" smd roundrect (at 0.25 -1.2625 90) (size 0.25 0.675) (layers "F.Cu" "F.Paste" "F.Mask") (roundrect_rratio 0.25) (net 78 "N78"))
  (pad "13" smd roundrect (at -0.25 -1.2625 90) (size 0.25 0.675) (layers "F.Cu" "F.Paste" "F.Mask") (roundrect_rratio 0.25) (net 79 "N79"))
  (pad "14" smd roundrect (at -0.75 -1.2625 90) (size 0.25 0.675) (layers "F.Cu" "F.Paste" "F.Mask") (roundrect_rratio 0.25) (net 73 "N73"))
  (pad "15" smd rect (at 0 0 90) (size 1.45 1.45) (layers "F.Cu" "F.Mask") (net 76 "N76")))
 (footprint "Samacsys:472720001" (layer "F.Cu") (at 23.19 47.84 -90)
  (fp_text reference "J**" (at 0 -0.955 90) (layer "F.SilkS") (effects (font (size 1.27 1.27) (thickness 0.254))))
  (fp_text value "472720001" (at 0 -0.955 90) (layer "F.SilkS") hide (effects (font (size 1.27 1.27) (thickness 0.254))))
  (pad "" np_thru_hole circle (at 0 2.99 270) (size 1.45 1.45) (drill 1.45) (layers "*.Cu" "*.Mask"))
  (pad "1" smd rect (at 5.5 -7.29 270) (size 0.28 2.4) (layers "F.Cu" "F.Paste" "F.Mask"))
  (pad "2" smd rect (at 5 -7.29 270) (size 0.28 2.4) (layers "F.Cu" "F.Paste" "F.Mask"))
  (pad "3" smd rect (at 4.5 -7.29 270) (size 0.28 2.4) (layers "F.Cu" "F.Paste" "F.Mask"))
  (pad "4" smd rect (at 4 -7.29 270) (size 0.28 2.4) (layers "F.Cu" "F.Paste" "F.Mask"))
  (pad "5" smd rect (at 3.5 -7.29 270) (size 0.28 2.4) (layers "F.Cu" "F.Paste" "F.Mask"))
  (pad "6" smd rect (at 3 -7.29 270) (size 0.28 2.4) (layers "F.Cu" "F.Paste" "F.Mask"))
  (pad "7" smd rect (at 2.5 -7.29 270) (size 0.28 2.4) (layers "F.Cu" "F.Paste" "F.Mask"))
  (pad "8" smd rect (at 2 -7.29 270) (size 0.28 2.4) (layers "F.Cu" "F.Paste" "F.Mask"))
  (pad "9" smd rect (at 1.5 -7.29 270) (size 0.28 2.4) (layers "F.Cu" "F.Paste" "F.Mask"))
  (pad "10" smd rect (at 1 -7.29 270) (size 0.28 2.4) (layers "F.Cu" "F.Paste" "F.Mask"))
  (pad "11" smd rect (at 0.5 -7.29 270) (size 0.28 2.4) (layers "F.Cu" "F.Paste" "F.Mask"))
  (pad "12" smd rect (at 0 -7.29 270) (size 0.28 2.4) (layers "F.Cu" "F.Paste" "F.Mask"))
  (pad "13" smd rect (at -0.5 -7.29 270) (size 0.28 2.4) (layers "F.Cu" "F.Paste" "F.Mask"))
  (pad "14" smd rect (at -1 -7.29 270) (size 0.28 2.4) (layers "F.Cu" "F.Paste" "F.Mask"))
  (pad "15" smd rect (at -1.5 -7.29 270) (size 0.28 2.4) (layers "F.Cu" "F.Paste" "F.Mask"))
  (pad "16" smd rect (at -2 -7.29 270) (size 0.28 2.4) (layers "F.Cu" "F.Paste" "F.Mask"))
  (pad "17" smd rect (at -2.5 -7.29 270) (size 0.28 2.4) (layers "F.Cu" "F.Paste" "F.Mask"))
  (pad "18" smd rect (at -3 -7.29 270) (size 0.28 2.4) (layers "F.Cu" "F.Paste" "F.Mask"))
  (pad "19" smd rect (at -3.5 -7.29 270) (size 0.28 2.4) (layers "F.Cu" "F.Paste" "F.Mask"))
  (pad "20" smd rect (at -4 -7.29 270) (size 0.28 2.4) (layers "F.Cu" "F.Paste" "F.Mask"))
  (pad "MH1" thru_hole circle (at -8.25 2.09 270) (size 1.98 1.98) (drill 1.32) (layers "*.Cu" "*.Mask"))
  (pad "MH2" thru_hole circle (at -8.25 -4.69 270) (size 2.655 2.655) (drill 1.77) (layers "*.Cu" "*.Mask"))
  (pad "MH3" thru_hole circle (at 8.25 -4.69 270) (size 2.655 2.655) (drill 1.77) (layers "*.Cu" "*.Mask"))
  (pad "MH4" thru_hole circle (at 8.25 2.09 270) (size 1.98 1.98) (drill 1.32) (layers "*.Cu" "*.Mask")))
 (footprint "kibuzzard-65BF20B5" (layer "F.Cu") (at 73.66 17.78)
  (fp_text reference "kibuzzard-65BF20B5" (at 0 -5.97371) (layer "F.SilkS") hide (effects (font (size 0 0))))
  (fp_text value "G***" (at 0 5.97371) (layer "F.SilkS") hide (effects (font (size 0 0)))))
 (gr_line (start 109.22 55.88) (end 109.22 40.64) (stroke (width 0.1) (type default)) (layer "Edge.Cuts"))
 (gr_line (start 91.44 38.1) (end 91.44 53.34) (stroke (width 0.1) (type default)) (layer "Edge.Cuts"))
 (gr_line (start 139.7 20.32) (end 127 12.7) (stroke (width 0.1) (type default)) (layer "Edge.Cuts"))
 (gr_line (start 109.22 40.64) (end 91.44 38.1) (stroke (width 0.1) (type default)) (layer "Edge.Cuts"))
 (gr_line (start 124.46 73.66) (end 139.7 20.32) (stroke (width 0.1) (type default)) (layer "Edge.Cuts"))
 (gr_line (start 12.7 12.7) (end 12.7 71.12) (stroke (width 0.1) (type default)) (layer "Edge.Cuts"))
 (gr_line (start 127 12.7) (end 12.7 12.7) (stroke (width 0.1) (type default)) (layer "Edge.Cuts"))
 (gr_line (start 12.7 71.12) (end 124.46 73.66) (stroke (width 0.1) (type default)) (layer "Edge.Cuts"))
 (gr_line (start 91.44 53.34) (end 109.22 55.88) (stroke (width 0.1) (type default)) (layer "Edge.Cuts"))
 (segment (start 50.785 34.56) (end 53.910784 34.56) (width 0.25) (layer "F.Cu") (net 2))
 (segment (start 53.910784 34.56) (end 54.353284 35.0025) (width 0.25) (layer "F.Cu") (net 2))
 (segment (start 54.166888 35.4525) (end 54.303284 35.4525) (width 0.25) (layer "F.Cu") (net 3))
 (segment (start 50.785 35.06) (end 53.774388 35.06) (width 0.25) (layer "F.Cu") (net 3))
 (segment (start 53.774388 35.06) (end 54.166888 35.4525) (width 0.25) (layer "F.Cu") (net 3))
 (segment (start 53.980492 35.9025) (end 54.253284 35.9025) (width 0.25) (layer "F.Cu") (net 4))
 (segment (start 53.637992 35.56) (end 53.980492 35.9025) (width 0.25) (layer "F.Cu") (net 4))
 (segment (start 50.785 35.56) (end 53.637992 35.56) (width 0.25) (layer "F.Cu") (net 4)))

